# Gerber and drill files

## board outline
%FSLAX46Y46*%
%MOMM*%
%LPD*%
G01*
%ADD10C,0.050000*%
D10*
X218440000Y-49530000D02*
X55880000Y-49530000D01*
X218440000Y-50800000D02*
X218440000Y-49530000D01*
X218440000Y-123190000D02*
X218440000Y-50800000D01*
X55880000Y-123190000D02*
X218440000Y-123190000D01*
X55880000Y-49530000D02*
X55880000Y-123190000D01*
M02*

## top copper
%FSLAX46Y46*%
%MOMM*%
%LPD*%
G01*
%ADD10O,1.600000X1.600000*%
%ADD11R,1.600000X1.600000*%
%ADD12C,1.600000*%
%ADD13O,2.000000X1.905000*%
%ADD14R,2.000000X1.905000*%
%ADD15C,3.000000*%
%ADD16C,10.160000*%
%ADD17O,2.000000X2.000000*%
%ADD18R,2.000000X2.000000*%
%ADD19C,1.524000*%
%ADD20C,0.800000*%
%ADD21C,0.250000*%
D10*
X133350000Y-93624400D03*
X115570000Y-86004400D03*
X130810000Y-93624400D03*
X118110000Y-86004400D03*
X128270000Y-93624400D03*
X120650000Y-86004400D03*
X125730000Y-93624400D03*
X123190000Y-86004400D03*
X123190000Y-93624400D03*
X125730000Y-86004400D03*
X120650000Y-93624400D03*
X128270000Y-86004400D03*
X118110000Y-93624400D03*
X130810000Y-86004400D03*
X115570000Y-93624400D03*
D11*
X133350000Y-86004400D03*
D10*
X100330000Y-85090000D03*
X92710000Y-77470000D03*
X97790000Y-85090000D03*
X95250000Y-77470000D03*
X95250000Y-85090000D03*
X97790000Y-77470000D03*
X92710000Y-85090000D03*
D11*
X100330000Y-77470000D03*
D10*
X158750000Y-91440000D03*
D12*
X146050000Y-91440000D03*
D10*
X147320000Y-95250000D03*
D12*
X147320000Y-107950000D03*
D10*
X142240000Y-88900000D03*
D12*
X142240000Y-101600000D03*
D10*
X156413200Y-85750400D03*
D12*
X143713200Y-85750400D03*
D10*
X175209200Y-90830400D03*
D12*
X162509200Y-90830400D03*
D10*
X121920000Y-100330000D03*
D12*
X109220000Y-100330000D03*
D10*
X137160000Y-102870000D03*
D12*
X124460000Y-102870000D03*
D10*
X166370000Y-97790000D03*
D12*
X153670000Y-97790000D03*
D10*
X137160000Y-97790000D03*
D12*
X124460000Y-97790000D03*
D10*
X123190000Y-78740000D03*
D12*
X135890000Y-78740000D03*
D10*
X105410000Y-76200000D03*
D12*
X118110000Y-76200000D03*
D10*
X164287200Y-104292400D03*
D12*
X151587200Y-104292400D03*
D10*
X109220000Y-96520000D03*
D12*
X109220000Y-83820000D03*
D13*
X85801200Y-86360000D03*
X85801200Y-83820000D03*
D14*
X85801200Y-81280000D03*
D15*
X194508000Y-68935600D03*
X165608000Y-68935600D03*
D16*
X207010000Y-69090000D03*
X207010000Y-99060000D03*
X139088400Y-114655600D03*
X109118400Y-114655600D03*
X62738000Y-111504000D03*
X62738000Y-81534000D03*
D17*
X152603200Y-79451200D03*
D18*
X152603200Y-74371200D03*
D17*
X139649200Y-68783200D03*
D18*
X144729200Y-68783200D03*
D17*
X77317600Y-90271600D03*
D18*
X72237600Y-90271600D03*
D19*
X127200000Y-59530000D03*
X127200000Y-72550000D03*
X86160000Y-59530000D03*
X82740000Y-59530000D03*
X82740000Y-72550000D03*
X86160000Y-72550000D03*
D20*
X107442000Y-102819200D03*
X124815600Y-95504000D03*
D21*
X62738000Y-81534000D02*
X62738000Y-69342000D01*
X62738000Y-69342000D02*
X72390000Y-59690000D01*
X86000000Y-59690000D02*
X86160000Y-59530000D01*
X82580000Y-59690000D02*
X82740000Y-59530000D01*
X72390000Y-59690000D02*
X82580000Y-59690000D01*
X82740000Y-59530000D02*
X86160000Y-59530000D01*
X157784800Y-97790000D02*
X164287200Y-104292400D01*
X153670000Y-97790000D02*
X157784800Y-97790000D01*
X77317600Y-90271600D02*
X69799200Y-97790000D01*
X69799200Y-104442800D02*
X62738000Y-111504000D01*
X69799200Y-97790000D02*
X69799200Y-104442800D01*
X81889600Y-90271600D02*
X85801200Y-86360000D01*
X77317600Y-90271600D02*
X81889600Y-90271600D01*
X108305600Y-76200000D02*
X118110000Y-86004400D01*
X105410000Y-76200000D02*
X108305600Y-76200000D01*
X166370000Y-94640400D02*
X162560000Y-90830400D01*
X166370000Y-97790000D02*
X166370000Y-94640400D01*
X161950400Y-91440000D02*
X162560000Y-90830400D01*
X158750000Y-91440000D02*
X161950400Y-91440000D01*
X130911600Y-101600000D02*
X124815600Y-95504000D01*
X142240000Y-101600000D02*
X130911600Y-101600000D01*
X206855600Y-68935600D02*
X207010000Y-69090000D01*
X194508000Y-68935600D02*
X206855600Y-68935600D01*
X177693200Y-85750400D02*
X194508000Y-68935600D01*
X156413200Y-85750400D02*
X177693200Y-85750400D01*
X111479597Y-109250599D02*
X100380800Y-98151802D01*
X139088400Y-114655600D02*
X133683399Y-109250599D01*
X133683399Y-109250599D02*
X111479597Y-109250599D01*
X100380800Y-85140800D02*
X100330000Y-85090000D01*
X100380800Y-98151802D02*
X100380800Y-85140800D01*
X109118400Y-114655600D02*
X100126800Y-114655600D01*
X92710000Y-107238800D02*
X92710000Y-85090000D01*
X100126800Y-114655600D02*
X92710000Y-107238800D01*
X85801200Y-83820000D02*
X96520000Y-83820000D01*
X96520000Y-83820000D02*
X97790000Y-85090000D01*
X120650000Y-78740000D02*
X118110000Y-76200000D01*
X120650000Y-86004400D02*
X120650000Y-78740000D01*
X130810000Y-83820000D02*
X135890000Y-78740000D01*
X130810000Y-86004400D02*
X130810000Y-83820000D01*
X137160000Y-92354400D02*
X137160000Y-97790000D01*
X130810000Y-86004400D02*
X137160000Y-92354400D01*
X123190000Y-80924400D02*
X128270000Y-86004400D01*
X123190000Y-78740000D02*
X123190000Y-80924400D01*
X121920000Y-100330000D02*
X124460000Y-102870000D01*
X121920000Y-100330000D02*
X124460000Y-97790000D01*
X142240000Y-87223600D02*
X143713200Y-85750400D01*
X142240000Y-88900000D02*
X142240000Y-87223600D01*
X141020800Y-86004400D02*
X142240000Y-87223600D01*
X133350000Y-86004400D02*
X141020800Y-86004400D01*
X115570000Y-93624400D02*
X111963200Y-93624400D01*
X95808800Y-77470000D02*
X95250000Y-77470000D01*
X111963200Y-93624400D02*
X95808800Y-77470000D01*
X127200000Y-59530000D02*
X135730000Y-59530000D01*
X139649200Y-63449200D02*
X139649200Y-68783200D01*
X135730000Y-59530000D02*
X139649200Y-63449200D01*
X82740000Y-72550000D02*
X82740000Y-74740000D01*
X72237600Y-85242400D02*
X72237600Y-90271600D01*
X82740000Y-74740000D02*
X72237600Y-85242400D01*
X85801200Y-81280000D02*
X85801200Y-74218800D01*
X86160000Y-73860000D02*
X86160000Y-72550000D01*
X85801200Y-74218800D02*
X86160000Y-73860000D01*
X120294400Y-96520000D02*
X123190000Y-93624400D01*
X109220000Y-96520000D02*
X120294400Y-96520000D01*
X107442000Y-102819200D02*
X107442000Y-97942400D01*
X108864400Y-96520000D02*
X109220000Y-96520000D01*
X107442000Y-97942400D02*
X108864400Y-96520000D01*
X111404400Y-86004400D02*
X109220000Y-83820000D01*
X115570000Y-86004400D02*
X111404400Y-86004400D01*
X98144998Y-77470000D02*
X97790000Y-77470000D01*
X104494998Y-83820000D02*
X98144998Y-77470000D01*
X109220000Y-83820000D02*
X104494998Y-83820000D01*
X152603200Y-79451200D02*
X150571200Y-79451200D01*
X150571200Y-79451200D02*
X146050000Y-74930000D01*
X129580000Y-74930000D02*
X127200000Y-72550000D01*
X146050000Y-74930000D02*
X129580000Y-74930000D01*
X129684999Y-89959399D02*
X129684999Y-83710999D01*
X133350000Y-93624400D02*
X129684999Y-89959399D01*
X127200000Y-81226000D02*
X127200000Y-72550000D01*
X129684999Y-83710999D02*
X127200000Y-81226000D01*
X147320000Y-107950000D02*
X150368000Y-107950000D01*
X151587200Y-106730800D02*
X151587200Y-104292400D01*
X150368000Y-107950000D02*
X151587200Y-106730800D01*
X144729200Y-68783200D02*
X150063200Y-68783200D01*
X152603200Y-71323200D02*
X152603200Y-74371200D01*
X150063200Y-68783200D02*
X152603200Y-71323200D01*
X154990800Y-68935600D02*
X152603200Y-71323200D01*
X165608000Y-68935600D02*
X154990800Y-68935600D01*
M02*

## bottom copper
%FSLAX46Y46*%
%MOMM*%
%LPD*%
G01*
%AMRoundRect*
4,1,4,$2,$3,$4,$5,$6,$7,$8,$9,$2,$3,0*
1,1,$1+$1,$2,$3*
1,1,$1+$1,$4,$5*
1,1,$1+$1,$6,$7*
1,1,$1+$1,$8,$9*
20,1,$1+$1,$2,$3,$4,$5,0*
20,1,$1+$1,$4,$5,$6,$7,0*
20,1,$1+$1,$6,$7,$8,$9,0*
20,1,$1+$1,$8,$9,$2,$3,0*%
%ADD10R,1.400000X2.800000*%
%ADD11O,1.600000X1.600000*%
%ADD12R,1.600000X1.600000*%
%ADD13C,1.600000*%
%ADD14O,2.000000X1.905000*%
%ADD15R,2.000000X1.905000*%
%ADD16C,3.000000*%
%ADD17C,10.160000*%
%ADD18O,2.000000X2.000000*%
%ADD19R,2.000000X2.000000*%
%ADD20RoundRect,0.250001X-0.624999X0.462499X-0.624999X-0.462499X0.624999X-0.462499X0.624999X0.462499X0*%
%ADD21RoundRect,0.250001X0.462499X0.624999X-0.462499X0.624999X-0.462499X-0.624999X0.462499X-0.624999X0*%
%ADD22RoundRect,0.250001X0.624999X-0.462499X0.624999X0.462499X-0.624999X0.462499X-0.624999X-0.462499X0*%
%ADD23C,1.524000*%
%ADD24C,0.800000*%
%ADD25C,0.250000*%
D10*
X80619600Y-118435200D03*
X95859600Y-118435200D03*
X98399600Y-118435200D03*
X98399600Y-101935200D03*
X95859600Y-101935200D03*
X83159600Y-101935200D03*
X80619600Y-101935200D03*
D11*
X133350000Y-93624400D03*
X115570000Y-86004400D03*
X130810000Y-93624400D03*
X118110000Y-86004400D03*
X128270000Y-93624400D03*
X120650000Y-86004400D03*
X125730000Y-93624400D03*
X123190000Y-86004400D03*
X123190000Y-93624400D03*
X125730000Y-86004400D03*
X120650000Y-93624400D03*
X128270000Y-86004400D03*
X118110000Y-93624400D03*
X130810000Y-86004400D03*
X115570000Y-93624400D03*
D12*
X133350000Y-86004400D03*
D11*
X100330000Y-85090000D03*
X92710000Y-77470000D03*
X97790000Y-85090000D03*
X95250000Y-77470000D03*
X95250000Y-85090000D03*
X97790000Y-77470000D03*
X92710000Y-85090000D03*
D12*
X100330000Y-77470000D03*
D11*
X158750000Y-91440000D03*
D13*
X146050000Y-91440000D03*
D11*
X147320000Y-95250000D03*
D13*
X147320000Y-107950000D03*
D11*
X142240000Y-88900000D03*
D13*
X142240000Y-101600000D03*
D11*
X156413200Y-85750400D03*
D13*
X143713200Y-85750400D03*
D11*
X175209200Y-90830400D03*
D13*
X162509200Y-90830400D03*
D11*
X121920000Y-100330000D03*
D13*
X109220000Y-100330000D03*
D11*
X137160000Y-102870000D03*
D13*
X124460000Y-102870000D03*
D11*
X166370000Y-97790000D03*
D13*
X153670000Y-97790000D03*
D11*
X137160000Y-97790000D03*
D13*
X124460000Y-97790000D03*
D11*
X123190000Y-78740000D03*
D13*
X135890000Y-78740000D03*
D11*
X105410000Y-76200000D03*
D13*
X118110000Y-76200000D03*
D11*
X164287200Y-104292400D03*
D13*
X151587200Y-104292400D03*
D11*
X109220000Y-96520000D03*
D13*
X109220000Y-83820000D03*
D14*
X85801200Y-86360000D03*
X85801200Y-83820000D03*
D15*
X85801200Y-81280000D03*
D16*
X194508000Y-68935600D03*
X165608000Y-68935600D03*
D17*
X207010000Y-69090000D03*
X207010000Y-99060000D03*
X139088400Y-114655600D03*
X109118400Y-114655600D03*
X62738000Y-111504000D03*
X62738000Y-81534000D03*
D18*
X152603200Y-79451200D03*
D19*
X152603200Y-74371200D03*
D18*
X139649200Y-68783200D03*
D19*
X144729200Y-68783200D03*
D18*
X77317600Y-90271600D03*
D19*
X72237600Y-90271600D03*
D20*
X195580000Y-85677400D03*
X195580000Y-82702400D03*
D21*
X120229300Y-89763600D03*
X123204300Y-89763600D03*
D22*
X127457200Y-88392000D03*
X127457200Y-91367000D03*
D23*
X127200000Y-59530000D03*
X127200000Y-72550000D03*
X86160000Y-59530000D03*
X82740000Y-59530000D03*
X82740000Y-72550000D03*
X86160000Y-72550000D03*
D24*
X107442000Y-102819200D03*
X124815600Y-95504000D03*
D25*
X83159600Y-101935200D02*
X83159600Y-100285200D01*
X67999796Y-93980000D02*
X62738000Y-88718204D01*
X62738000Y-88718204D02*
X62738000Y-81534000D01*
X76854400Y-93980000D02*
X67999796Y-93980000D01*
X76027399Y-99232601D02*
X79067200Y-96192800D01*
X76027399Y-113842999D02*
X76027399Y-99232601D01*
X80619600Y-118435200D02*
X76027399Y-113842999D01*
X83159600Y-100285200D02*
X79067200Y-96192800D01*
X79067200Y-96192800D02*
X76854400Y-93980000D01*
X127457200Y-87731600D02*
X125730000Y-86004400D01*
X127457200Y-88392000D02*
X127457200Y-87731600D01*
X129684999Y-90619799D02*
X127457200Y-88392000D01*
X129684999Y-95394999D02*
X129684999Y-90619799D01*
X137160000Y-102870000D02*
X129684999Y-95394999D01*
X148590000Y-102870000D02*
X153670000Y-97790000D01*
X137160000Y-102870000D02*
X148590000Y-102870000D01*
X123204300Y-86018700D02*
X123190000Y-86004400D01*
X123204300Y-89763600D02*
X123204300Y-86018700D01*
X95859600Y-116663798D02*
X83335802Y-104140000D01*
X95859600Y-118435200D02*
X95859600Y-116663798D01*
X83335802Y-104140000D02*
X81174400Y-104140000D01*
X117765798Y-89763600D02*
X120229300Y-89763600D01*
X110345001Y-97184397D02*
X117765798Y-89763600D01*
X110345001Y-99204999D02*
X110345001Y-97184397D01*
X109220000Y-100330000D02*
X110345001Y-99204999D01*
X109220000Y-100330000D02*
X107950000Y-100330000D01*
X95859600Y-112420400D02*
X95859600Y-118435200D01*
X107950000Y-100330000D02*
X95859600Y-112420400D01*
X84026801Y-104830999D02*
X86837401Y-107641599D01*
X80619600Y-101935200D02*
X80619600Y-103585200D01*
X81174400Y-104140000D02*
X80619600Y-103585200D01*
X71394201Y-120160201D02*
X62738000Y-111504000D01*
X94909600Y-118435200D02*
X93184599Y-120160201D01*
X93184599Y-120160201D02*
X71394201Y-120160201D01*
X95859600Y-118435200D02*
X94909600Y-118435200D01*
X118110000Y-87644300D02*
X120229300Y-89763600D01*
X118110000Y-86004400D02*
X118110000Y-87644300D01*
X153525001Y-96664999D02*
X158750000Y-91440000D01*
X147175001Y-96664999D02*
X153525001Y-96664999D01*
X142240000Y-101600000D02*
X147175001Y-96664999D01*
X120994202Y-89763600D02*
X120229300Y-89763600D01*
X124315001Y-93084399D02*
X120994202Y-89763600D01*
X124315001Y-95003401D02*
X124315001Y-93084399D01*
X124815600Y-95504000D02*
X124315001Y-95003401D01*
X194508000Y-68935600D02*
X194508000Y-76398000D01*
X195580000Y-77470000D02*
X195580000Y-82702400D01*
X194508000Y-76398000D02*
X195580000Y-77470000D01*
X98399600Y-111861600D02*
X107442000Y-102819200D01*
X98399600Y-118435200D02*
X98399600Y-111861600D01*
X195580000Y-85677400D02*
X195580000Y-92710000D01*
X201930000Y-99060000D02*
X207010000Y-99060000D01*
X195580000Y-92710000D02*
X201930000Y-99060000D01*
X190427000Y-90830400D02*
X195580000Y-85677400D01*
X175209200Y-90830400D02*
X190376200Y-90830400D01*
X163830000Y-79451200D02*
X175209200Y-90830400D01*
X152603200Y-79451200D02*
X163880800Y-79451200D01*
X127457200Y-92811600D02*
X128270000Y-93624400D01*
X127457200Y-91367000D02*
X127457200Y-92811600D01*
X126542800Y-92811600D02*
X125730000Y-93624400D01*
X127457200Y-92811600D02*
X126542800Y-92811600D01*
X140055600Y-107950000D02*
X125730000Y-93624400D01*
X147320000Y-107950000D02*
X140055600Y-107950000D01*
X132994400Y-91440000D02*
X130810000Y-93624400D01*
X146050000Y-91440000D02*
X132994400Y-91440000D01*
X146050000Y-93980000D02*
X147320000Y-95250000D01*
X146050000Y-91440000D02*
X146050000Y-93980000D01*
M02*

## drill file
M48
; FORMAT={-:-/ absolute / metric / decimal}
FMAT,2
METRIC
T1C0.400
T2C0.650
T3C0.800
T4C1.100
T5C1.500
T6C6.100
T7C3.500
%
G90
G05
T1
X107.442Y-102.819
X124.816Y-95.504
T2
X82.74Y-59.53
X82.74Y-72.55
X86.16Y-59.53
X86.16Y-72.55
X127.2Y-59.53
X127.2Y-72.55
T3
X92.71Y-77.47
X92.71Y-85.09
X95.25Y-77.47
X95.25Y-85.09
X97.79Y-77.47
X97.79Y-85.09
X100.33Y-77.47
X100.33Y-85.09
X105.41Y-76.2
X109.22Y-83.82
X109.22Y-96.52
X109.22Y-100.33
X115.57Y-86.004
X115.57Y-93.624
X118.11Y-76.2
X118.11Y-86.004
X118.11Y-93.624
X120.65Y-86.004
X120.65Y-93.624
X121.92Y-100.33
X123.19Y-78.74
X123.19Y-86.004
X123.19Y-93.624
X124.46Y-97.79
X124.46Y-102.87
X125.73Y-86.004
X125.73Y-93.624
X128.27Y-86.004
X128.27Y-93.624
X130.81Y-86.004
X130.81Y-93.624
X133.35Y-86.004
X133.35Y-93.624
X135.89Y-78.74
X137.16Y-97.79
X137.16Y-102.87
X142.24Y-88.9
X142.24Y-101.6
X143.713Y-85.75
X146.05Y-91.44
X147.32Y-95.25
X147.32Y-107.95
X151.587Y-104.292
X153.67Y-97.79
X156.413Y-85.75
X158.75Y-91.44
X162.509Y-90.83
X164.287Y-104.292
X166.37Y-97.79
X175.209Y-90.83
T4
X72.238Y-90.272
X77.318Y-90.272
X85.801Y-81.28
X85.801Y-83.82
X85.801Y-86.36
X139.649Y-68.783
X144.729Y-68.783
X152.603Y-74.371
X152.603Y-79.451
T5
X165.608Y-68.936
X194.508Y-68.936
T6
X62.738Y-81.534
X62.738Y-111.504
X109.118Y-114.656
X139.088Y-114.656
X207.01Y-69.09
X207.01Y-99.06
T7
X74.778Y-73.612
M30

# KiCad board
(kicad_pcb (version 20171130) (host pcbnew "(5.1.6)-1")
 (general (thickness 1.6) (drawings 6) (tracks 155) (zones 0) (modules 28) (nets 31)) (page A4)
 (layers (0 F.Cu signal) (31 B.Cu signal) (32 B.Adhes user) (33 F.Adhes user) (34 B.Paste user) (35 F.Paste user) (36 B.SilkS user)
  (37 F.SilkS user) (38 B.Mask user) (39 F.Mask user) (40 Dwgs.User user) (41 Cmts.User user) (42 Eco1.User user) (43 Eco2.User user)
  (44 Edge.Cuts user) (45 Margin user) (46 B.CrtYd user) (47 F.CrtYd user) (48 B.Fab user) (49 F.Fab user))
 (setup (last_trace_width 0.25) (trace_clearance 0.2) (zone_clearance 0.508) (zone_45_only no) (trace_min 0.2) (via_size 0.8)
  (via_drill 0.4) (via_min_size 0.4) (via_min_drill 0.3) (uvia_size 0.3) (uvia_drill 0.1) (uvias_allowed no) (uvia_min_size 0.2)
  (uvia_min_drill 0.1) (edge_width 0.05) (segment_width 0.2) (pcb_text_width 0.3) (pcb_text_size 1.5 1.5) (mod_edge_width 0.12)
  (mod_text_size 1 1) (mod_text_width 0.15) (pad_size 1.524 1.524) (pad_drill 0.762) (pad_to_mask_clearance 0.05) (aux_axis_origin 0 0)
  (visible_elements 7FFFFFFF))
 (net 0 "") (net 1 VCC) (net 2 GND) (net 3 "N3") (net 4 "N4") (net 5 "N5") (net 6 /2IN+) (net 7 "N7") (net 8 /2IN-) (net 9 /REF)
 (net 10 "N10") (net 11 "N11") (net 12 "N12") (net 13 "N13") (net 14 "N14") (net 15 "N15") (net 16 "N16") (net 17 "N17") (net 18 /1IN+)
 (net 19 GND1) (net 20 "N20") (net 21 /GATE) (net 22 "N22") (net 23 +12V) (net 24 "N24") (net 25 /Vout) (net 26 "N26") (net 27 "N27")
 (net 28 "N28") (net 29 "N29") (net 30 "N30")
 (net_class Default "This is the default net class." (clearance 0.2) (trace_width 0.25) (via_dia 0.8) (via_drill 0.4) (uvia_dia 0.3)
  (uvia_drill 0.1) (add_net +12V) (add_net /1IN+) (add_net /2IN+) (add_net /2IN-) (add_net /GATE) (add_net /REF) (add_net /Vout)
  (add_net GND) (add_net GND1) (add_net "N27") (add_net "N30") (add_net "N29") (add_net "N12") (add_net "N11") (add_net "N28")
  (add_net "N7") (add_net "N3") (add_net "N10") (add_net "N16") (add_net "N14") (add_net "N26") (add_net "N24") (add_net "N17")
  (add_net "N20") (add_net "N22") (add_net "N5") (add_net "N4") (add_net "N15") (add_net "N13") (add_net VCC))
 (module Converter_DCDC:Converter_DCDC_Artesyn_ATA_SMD (layer B.Cu) (at 89.5096 110.1852 270)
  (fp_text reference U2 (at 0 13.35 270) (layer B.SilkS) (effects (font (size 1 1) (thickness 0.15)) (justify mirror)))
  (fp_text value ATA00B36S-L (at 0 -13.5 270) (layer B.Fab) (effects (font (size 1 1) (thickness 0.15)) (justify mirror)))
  (pad 16 smd rect (at 8.25 8.89 270) (size 2.8 1.4) (layers B.Cu B.Paste B.Mask) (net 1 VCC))
  (pad 10 smd rect (at 8.25 -6.35 270) (size 2.8 1.4) (layers B.Cu B.Paste B.Mask) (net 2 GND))
  (pad 9 smd rect (at 8.25 -8.89 270) (size 2.8 1.4) (layers B.Cu B.Paste B.Mask) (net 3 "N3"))
  (pad 8 smd rect (at -8.25 -8.89 270) (size 2.8 1.4) (layers B.Cu B.Paste B.Mask) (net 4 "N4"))
  (pad 7 smd rect (at -8.25 -6.35 270) (size 2.8 1.4) (layers B.Cu B.Paste B.Mask) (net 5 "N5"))
  (pad 2 smd rect (at -8.25 6.35 270) (size 2.8 1.4) (layers B.Cu B.Paste B.Mask) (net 1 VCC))
  (pad 1 smd rect (at -8.25 8.89 270) (size 2.8 1.4) (layers B.Cu B.Paste B.Mask) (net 2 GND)))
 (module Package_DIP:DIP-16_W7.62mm (layer F.Cu) (at 133.35 86.0044 270)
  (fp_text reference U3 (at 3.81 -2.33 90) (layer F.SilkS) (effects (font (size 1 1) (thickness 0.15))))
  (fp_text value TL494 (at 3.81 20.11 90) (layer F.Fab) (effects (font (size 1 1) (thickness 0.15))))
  (pad 16 thru_hole oval (at 7.62 0 270) (size 1.6 1.6) (drill 0.8) (layers *.Cu *.Mask) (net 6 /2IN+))
  (pad 8 thru_hole oval (at 0 17.78 270) (size 1.6 1.6) (drill 0.8) (layers *.Cu *.Mask) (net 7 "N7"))
  (pad 15 thru_hole oval (at 7.62 2.54 270) (size 1.6 1.6) (drill 0.8) (layers *.Cu *.Mask) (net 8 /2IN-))
  (pad 7 thru_hole oval (at 0 15.24 270) (size 1.6 1.6) (drill 0.8) (layers *.Cu *.Mask) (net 2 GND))
  (pad 14 thru_hole oval (at 7.62 5.08 270) (size 1.6 1.6) (drill 0.8) (layers *.Cu *.Mask) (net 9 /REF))
  (pad 6 thru_hole oval (at 0 12.7 270) (size 1.6 1.6) (drill 0.8) (layers *.Cu *.Mask) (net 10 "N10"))
  (pad 13 thru_hole oval (at 7.62 7.62 270) (size 1.6 1.6) (drill 0.8) (layers *.Cu *.Mask) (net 9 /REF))
  (pad 5 thru_hole oval (at 0 10.16 270) (size 1.6 1.6) (drill 0.8) (layers *.Cu *.Mask) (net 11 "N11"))
  (pad 12 thru_hole oval (at 7.62 10.16 270) (size 1.6 1.6) (drill 0.8) (layers *.Cu *.Mask) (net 3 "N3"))
  (pad 4 thru_hole oval (at 0 7.62 270) (size 1.6 1.6) (drill 0.8) (layers *.Cu *.Mask) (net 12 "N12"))
  (pad 11 thru_hole oval (at 7.62 12.7 270) (size 1.6 1.6) (drill 0.8) (layers *.Cu *.Mask) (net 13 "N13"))
  (pad 3 thru_hole oval (at 0 5.08 270) (size 1.6 1.6) (drill 0.8) (layers *.Cu *.Mask) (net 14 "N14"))
  (pad 10 thru_hole oval (at 7.62 15.24 270) (size 1.6 1.6) (drill 0.8) (layers *.Cu *.Mask) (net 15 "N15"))
  (pad 2 thru_hole oval (at 0 2.54 270) (size 1.6 1.6) (drill 0.8) (layers *.Cu *.Mask) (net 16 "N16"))
  (pad 9 thru_hole oval (at 7.62 17.78 270) (size 1.6 1.6) (drill 0.8) (layers *.Cu *.Mask) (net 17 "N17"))
  (pad 1 thru_hole rect (at 0 0 270) (size 1.6 1.6) (drill 0.8) (layers *.Cu *.Mask) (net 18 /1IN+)))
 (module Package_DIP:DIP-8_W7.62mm (layer F.Cu) (at 100.33 77.47 270)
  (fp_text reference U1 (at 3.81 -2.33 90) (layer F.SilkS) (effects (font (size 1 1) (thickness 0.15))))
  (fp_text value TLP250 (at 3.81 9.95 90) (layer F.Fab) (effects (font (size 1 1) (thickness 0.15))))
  (pad 8 thru_hole oval (at 7.62 0 270) (size 1.6 1.6) (drill 0.8) (layers *.Cu *.Mask) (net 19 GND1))
  (pad 4 thru_hole oval (at 0 7.62 270) (size 1.6 1.6) (drill 0.8) (layers *.Cu *.Mask) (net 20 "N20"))
  (pad 7 thru_hole oval (at 7.62 2.54 270) (size 1.6 1.6) (drill 0.8) (layers *.Cu *.Mask) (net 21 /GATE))
  (pad 3 thru_hole oval (at 0 5.08 270) (size 1.6 1.6) (drill 0.8) (layers *.Cu *.Mask) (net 17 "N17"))
  (pad 6 thru_hole oval (at 7.62 5.08 270) (size 1.6 1.6) (drill 0.8) (layers *.Cu *.Mask) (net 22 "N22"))
  (pad 2 thru_hole oval (at 0 2.54 270) (size 1.6 1.6) (drill 0.8) (layers *.Cu *.Mask) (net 7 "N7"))
  (pad 5 thru_hole oval (at 7.62 7.62 270) (size 1.6 1.6) (drill 0.8) (layers *.Cu *.Mask) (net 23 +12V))
  (pad 1 thru_hole rect (at 0 0 270) (size 1.6 1.6) (drill 0.8) (layers *.Cu *.Mask) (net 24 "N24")))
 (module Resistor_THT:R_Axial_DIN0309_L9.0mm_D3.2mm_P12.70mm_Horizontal (layer F.Cu) (at 146.05 91.44)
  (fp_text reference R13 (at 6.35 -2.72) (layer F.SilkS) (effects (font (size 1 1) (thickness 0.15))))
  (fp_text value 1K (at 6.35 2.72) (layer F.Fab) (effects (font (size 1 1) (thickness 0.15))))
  (pad 2 thru_hole oval (at 12.7 0) (size 1.6 1.6) (drill 0.8) (layers *.Cu *.Mask) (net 2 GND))
  (pad 1 thru_hole circle (at 0 0) (size 1.6 1.6) (drill 0.8) (layers *.Cu *.Mask) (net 8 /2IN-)))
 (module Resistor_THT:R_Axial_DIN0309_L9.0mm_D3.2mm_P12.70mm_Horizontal (layer F.Cu) (at 147.32 107.95 90)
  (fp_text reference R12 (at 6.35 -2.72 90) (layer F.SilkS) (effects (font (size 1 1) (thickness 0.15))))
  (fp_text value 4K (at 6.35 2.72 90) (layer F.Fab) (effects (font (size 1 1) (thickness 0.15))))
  (pad 2 thru_hole oval (at 12.7 0 90) (size 1.6 1.6) (drill 0.8) (layers *.Cu *.Mask) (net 8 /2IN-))
  (pad 1 thru_hole circle (at 0 0 90) (size 1.6 1.6) (drill 0.8) (layers *.Cu *.Mask) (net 9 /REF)))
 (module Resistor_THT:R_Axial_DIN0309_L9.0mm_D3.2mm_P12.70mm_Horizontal (layer F.Cu) (at 142.24 101.6 90)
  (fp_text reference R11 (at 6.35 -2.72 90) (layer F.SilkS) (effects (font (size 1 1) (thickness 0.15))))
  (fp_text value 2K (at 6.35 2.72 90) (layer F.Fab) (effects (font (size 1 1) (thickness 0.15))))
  (pad 2 thru_hole oval (at 12.7 0 90) (size 1.6 1.6) (drill 0.8) (layers *.Cu *.Mask) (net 18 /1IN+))
  (pad 1 thru_hole circle (at 0 0 90) (size 1.6 1.6) (drill 0.8) (layers *.Cu *.Mask) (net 2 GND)))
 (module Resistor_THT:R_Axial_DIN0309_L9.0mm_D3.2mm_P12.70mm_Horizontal (layer F.Cu) (at 143.7132 85.7504)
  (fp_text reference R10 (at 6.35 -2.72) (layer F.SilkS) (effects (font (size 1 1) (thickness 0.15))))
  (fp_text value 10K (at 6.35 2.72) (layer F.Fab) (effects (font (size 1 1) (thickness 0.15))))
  (pad 2 thru_hole oval (at 12.7 0) (size 1.6 1.6) (drill 0.8) (layers *.Cu *.Mask) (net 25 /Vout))
  (pad 1 thru_hole circle (at 0 0) (size 1.6 1.6) (drill 0.8) (layers *.Cu *.Mask) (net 18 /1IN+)))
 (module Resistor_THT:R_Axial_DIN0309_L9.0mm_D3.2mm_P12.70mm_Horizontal (layer F.Cu) (at 162.5092 90.8304)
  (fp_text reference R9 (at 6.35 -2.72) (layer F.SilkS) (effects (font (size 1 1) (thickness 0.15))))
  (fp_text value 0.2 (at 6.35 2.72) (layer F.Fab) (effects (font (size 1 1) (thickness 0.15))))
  (pad 2 thru_hole oval (at 12.7 0) (size 1.6 1.6) (drill 0.8) (layers *.Cu *.Mask) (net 6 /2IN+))
  (pad 1 thru_hole circle (at 0 0) (size 1.6 1.6) (drill 0.8) (layers *.Cu *.Mask) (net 2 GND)))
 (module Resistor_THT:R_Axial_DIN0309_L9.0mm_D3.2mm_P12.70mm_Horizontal (layer F.Cu) (at 109.22 100.33)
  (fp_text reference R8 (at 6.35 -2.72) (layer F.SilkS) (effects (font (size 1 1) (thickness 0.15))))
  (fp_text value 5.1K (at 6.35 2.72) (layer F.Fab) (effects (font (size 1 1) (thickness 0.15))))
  (pad 2 thru_hole oval (at 12.7 0) (size 1.6 1.6) (drill 0.8) (layers *.Cu *.Mask) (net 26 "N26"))
  (pad 1 thru_hole circle (at 0 0) (size 1.6 1.6) (drill 0.8) (layers *.Cu *.Mask) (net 2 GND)))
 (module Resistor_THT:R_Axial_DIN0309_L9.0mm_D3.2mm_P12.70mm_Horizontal (layer F.Cu) (at 124.46 102.87)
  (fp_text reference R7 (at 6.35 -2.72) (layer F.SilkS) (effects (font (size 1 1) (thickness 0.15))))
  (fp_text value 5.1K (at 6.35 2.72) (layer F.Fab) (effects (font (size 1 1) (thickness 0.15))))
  (pad 2 thru_hole oval (at 12.7 0) (size 1.6 1.6) (drill 0.8) (layers *.Cu *.Mask) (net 12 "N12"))
  (pad 1 thru_hole circle (at 0 0) (size 1.6 1.6) (drill 0.8) (layers *.Cu *.Mask) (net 26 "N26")))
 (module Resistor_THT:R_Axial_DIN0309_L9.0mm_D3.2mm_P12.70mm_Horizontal (layer F.Cu) (at 153.67 97.79)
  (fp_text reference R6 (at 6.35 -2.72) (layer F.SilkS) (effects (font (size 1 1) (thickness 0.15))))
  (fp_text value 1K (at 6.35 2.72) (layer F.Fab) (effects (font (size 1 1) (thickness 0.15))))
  (pad 2 thru_hole oval (at 12.7 0) (size 1.6 1.6) (drill 0.8) (layers *.Cu *.Mask) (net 2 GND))
  (pad 1 thru_hole circle (at 0 0) (size 1.6 1.6) (drill 0.8) (layers *.Cu *.Mask) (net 12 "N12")))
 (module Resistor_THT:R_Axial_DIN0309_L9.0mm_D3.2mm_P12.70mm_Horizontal (layer F.Cu) (at 124.46 97.79)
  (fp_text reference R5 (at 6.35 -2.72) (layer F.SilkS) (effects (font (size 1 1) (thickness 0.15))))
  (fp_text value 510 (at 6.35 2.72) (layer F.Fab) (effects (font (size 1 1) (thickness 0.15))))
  (pad 2 thru_hole oval (at 12.7 0) (size 1.6 1.6) (drill 0.8) (layers *.Cu *.Mask) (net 16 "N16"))
  (pad 1 thru_hole circle (at 0 0) (size 1.6 1.6) (drill 0.8) (layers *.Cu *.Mask) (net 26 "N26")))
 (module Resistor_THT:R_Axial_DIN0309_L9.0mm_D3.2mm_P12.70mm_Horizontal (layer F.Cu) (at 135.89 78.74 180)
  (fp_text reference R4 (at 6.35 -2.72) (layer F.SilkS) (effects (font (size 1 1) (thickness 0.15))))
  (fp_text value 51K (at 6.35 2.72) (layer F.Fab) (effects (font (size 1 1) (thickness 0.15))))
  (pad 2 thru_hole oval (at 12.7 0 180) (size 1.6 1.6) (drill 0.8) (layers *.Cu *.Mask) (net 14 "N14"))
  (pad 1 thru_hole circle (at 0 0 180) (size 1.6 1.6) (drill 0.8) (layers *.Cu *.Mask) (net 16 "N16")))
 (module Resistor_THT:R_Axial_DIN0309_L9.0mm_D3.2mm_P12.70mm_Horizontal (layer F.Cu) (at 118.11 76.2 180)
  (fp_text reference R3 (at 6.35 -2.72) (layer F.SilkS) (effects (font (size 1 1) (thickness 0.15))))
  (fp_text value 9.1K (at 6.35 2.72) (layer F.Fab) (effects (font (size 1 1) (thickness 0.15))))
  (pad 2 thru_hole oval (at 12.7 0 180) (size 1.6 1.6) (drill 0.8) (layers *.Cu *.Mask) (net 2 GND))
  (pad 1 thru_hole circle (at 0 0 180) (size 1.6 1.6) (drill 0.8) (layers *.Cu *.Mask) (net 10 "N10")))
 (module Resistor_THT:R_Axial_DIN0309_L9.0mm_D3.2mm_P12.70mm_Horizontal (layer F.Cu) (at 151.5872 104.2924)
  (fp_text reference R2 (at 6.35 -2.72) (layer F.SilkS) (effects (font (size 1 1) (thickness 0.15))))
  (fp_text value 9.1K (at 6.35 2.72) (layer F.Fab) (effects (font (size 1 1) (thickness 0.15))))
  (pad 2 thru_hole oval (at 12.7 0) (size 1.6 1.6) (drill 0.8) (layers *.Cu *.Mask) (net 12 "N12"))
  (pad 1 thru_hole circle (at 0 0) (size 1.6 1.6) (drill 0.8) (layers *.Cu *.Mask) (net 9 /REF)))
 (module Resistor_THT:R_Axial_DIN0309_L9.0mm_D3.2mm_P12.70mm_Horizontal (layer B.Cu) (at 109.22 83.82 270)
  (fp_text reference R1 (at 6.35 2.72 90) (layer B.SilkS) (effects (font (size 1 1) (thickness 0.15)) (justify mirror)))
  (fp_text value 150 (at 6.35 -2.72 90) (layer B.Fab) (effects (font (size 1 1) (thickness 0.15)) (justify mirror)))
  (pad 2 thru_hole oval (at 12.7 0 270) (size 1.6 1.6) (drill 0.8) (layers *.Cu *.Mask) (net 3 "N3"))
  (pad 1 thru_hole circle (at 0 0 270) (size 1.6 1.6) (drill 0.8) (layers *.Cu *.Mask) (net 7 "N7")))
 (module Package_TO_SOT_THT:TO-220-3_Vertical (layer F.Cu) (at 85.8012 81.28 270)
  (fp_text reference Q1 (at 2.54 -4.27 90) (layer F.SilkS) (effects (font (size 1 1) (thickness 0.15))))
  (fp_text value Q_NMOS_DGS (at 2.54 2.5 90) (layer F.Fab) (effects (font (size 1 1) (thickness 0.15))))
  (pad 3 thru_hole oval (at 5.08 0 270) (size 1.905 2) (drill 1.1) (layers *.Cu *.Mask) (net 2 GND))
  (pad 2 thru_hole oval (at 2.54 0 270) (size 1.905 2) (drill 1.1) (layers *.Cu *.Mask) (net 21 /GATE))
  (pad 1 thru_hole rect (at 0 0 270) (size 1.905 2) (drill 1.1) (layers *.Cu *.Mask) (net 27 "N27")))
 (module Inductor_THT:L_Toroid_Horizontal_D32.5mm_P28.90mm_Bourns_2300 (layer F.Cu) (at 165.608 68.9356)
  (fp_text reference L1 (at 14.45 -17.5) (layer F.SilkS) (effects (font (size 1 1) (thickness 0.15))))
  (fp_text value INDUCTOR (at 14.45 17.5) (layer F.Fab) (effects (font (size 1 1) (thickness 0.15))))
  (pad 2 thru_hole circle (at 28.9 0) (size 3 3) (drill 1.5) (layers *.Cu *.Mask) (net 25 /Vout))
  (pad 1 thru_hole circle (at 0 0) (size 3 3) (drill 1.5) (layers *.Cu *.Mask) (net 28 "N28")))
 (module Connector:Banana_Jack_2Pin (layer F.Cu) (at 207.01 99.06 90)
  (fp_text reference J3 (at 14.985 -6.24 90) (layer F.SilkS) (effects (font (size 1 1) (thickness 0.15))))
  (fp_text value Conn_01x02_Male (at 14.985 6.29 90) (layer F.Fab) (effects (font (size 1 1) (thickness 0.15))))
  (pad 2 thru_hole circle (at 29.97 0 90) (size 10.16 10.16) (drill 6.1) (layers *.Cu *.Mask) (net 25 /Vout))
  (pad 1 thru_hole circle (at 0 0 90) (size 10.16 10.16) (drill 6.1) (layers *.Cu *.Mask) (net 6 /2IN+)))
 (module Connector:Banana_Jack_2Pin (layer F.Cu) (at 109.1184 114.6556)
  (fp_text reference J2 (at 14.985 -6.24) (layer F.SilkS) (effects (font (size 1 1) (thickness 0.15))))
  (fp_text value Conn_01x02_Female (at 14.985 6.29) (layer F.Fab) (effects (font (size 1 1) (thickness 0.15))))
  (pad 2 thru_hole circle (at 29.97 0) (size 10.16 10.16) (drill 6.1) (layers *.Cu *.Mask) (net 19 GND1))
  (pad 1 thru_hole circle (at 0 0) (size 10.16 10.16) (drill 6.1) (layers *.Cu *.Mask) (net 23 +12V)))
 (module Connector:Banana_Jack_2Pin (layer F.Cu) (at 62.738 81.534 270)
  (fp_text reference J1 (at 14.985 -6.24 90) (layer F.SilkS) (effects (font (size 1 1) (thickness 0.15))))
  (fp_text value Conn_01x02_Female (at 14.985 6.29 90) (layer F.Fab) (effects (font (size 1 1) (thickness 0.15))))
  (pad 2 thru_hole circle (at 29.97 0 270) (size 10.16 10.16) (drill 6.1) (layers *.Cu *.Mask) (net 2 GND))
  (pad 1 thru_hole circle (at 0 0 270) (size 10.16 10.16) (drill 6.1) (layers *.Cu *.Mask) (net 1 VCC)))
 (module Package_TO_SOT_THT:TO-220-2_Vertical (layer F.Cu) (at 152.6032 74.3712 270)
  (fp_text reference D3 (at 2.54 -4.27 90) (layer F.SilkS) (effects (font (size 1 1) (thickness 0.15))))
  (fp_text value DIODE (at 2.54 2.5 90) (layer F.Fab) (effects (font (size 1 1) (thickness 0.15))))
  (pad 2 thru_hole oval (at 5.08 0 270) (size 2 2) (drill 1.1) (layers *.Cu *.Mask) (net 6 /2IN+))
  (pad 1 thru_hole rect (at 0 0 270) (size 2 2) (drill 1.1) (layers *.Cu *.Mask) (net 28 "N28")))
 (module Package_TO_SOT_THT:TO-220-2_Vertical (layer F.Cu) (at 144.7292 68.7832 180)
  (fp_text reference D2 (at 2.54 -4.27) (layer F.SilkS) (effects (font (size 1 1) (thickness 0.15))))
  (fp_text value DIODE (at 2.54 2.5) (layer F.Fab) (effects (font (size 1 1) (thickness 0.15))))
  (pad 2 thru_hole oval (at 5.08 0 180) (size 2 2) (drill 1.1) (layers *.Cu *.Mask) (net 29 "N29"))
  (pad 1 thru_hole rect (at 0 0 180) (size 2 2) (drill 1.1) (layers *.Cu *.Mask) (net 28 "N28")))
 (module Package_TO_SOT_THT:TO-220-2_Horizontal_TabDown (layer F.Cu) (at 72.2376 90.2716)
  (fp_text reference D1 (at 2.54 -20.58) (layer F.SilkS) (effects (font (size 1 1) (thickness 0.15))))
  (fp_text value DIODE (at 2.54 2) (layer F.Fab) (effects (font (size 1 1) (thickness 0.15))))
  (pad 2 thru_hole oval (at 5.08 0) (size 2 2) (drill 1.1) (layers *.Cu *.Mask) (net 2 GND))
  (pad 1 thru_hole rect (at 0 0) (size 2 2) (drill 1.1) (layers *.Cu *.Mask) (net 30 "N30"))
  (pad "" np_thru_hole oval (at 2.54 -16.66) (size 3.5 3.5) (drill 3.5) (layers *.Cu *.Mask)))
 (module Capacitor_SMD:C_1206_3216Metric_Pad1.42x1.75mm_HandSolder (layer B.Cu) (at 195.58 84.1899 270)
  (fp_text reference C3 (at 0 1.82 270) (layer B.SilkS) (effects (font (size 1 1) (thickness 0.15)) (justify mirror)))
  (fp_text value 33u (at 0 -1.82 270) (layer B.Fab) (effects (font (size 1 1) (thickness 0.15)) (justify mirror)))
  (pad 2 smd roundrect (at 1.4875 0 270) (size 1.425 1.75) (layers B.Cu B.Paste B.Mask) (roundrect_rratio 0.175439) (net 6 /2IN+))
  (pad 1 smd roundrect (at -1.4875 0 270) (size 1.425 1.75) (layers B.Cu B.Paste B.Mask) (roundrect_rratio 0.175439) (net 25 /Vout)))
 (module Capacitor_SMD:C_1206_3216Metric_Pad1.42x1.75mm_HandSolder (layer B.Cu) (at 121.7168 89.7636 180)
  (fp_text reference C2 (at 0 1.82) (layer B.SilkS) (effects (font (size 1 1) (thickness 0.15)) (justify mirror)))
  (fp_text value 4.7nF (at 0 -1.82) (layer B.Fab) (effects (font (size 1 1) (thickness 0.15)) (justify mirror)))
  (pad 2 smd roundrect (at 1.4875 0 180) (size 1.425 1.75) (layers B.Cu B.Paste B.Mask) (roundrect_rratio 0.175439) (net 2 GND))
  (pad 1 smd roundrect (at -1.4875 0 180) (size 1.425 1.75) (layers B.Cu B.Paste B.Mask) (roundrect_rratio 0.175439) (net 11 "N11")))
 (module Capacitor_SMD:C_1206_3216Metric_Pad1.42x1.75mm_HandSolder (layer B.Cu) (at 127.4572 89.8795 90)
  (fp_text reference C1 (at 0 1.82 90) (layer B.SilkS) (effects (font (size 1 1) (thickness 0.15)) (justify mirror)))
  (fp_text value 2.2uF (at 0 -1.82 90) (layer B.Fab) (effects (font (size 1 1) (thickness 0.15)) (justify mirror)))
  (pad 2 smd roundrect (at 1.4875 0 90) (size 1.425 1.75) (layers B.Cu B.Paste B.Mask) (roundrect_rratio 0.175439) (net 12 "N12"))
  (pad 1 smd roundrect (at -1.4875 0 90) (size 1.425 1.75) (layers B.Cu B.Paste B.Mask) (roundrect_rratio 0.175439) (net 9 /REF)))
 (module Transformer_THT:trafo (layer F.Cu) (at 106.68 66.04 90)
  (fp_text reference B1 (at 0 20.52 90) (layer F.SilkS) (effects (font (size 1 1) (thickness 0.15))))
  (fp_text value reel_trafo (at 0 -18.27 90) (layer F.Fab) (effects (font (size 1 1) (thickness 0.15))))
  (pad 6 thru_hole circle (at 6.51 20.52 90) (size 1.524 1.524) (drill 0.65) (layers *.Cu *.Mask) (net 29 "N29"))
  (pad 5 thru_hole circle (at -6.51 20.52 90) (size 1.524 1.524) (drill 0.65) (layers *.Cu *.Mask) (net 6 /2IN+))
  (pad 4 thru_hole circle (at 6.51 -20.52 90) (size 1.524 1.524) (drill 0.65) (layers *.Cu *.Mask) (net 1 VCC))
  (pad 3 thru_hole circle (at 6.51 -23.94 90) (size 1.524 1.524) (drill 0.65) (layers *.Cu *.Mask) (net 1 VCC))
  (pad 2 thru_hole circle (at -6.51 -23.94 90) (size 1.524 1.524) (drill 0.65) (layers *.Cu *.Mask) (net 30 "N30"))
  (pad 1 thru_hole circle (at -6.51 -20.52 90) (size 1.524 1.524) (drill 0.65) (layers *.Cu *.Mask) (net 27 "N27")))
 (gr_line (start 218.44 49.53) (end 55.88 49.53) (layer Edge.Cuts) (width 0.05))
 (gr_line (start 218.44 50.8) (end 218.44 49.53) (layer Edge.Cuts) (width 0.05))
 (gr_line (start 218.44 123.19) (end 218.44 50.8) (layer Edge.Cuts) (width 0.05))
 (gr_line (start 55.88 123.19) (end 218.44 123.19) (layer Edge.Cuts) (width 0.05))
 (gr_line (start 55.88 49.53) (end 55.88 123.19) (layer Edge.Cuts) (width 0.05))
 (via (at 107.442 102.8192) (size 0.8) (drill 0.4) (layers F.Cu B.Cu) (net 3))
 (via (at 124.8156 95.504) (size 0.8) (drill 0.4) (layers F.Cu B.Cu) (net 2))
 (segment (start 62.738 81.534) (end 62.738 69.342) (width 0.25) (layer F.Cu) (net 1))
 (segment (start 62.738 69.342) (end 72.39 59.69) (width 0.25) (layer F.Cu) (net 1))
 (segment (start 86 59.69) (end 86.16 59.53) (width 0.25) (layer F.Cu) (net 1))
 (segment (start 82.58 59.69) (end 82.74 59.53) (width 0.25) (layer F.Cu) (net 1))
 (segment (start 72.39 59.69) (end 82.58 59.69) (width 0.25) (layer F.Cu) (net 1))
 (segment (start 82.74 59.53) (end 86.16 59.53) (width 0.25) (layer F.Cu) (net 1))
 (segment (start 83.1596 101.9352) (end 83.1596 100.2852) (width 0.25) (layer B.Cu) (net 1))
 (segment (start 67.999796 93.98) (end 62.738 88.718204) (width 0.25) (layer B.Cu) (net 1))
 (segment (start 62.738 88.718204) (end 62.738 81.534) (width 0.25) (layer B.Cu) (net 1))
 (segment (start 76.8544 93.98) (end 67.999796 93.98) (width 0.25) (layer B.Cu) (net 1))
 (segment (start 76.027399 99.232601) (end 79.0672 96.1928) (width 0.25) (layer B.Cu) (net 1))
 (segment (start 76.027399 113.842999) (end 76.027399 99.232601) (width 0.25) (layer B.Cu) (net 1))
 (segment (start 80.6196 118.4352) (end 76.027399 113.842999) (width 0.25) (layer B.Cu) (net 1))
 (segment (start 83.1596 100.2852) (end 79.0672 96.1928) (width 0.25) (layer B.Cu) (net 1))
 (segment (start 79.0672 96.1928) (end 76.8544 93.98) (width 0.25) (layer B.Cu) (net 1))
 (segment (start 127.4572 87.7316) (end 125.73 86.0044) (width 0.25) (layer B.Cu) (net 12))
 (segment (start 127.4572 88.392) (end 127.4572 87.7316) (width 0.25) (layer B.Cu) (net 12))
 (segment (start 157.7848 97.79) (end 164.2872 104.2924) (width 0.25) (layer F.Cu) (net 12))
 (segment (start 153.67 97.79) (end 157.7848 97.79) (width 0.25) (layer F.Cu) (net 12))
 (segment (start 129.684999 90.619799) (end 127.4572 88.392) (width 0.25) (layer B.Cu) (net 12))
 (segment (start 129.684999 95.394999) (end 129.684999 90.619799) (width 0.25) (layer B.Cu) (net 12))
 (segment (start 137.16 102.87) (end 129.684999 95.394999) (width 0.25) (layer B.Cu) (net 12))
 (segment (start 148.59 102.87) (end 153.67 97.79) (width 0.25) (layer B.Cu) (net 12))
 (segment (start 137.16 102.87) (end 148.59 102.87) (width 0.25) (layer B.Cu) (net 12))
 (segment (start 123.2043 86.0187) (end 123.19 86.0044) (width 0.25) (layer B.Cu) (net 11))
 (segment (start 123.2043 89.7636) (end 123.2043 86.0187) (width 0.25) (layer B.Cu) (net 11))
 (segment (start 77.3176 90.2716) (end 69.7992 97.79) (width 0.25) (layer F.Cu) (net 2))
 (segment (start 69.7992 104.4428) (end 62.738 111.504) (width 0.25) (layer F.Cu) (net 2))
 (segment (start 69.7992 97.79) (end 69.7992 104.4428) (width 0.25) (layer F.Cu) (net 2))
 (segment (start 81.8896 90.2716) (end 85.8012 86.36) (width 0.25) (layer F.Cu) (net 2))
 (segment (start 77.3176 90.2716) (end 81.8896 90.2716) (width 0.25) (layer F.Cu) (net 2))
 (segment (start 95.8596 116.663798) (end 83.335802 104.14) (width 0.25) (layer B.Cu) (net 2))
 (segment (start 95.8596 118.4352) (end 95.8596 116.663798) (width 0.25) (layer B.Cu) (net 2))
 (segment (start 83.335802 104.14) (end 81.1744 104.14) (width 0.25) (layer B.Cu) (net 2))
 (segment (start 117.765798 89.7636) (end 120.2293 89.7636) (width 0.25) (layer B.Cu) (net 2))
 (segment (start 110.345001 97.184397) (end 117.765798 89.7636) (width 0.25) (layer B.Cu) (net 2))
 (segment (start 110.345001 99.204999) (end 110.345001 97.184397) (width 0.25) (layer B.Cu) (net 2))
 (segment (start 109.22 100.33) (end 110.345001 99.204999) (width 0.25) (layer B.Cu) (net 2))
 (segment (start 109.22 100.33) (end 107.95 100.33) (width 0.25) (layer B.Cu) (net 2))
 (segment (start 95.8596 112.4204) (end 95.8596 118.4352) (width 0.25) (layer B.Cu) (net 2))
 (segment (start 107.95 100.33) (end 95.8596 112.4204) (width 0.25) (layer B.Cu) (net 2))
 (segment (start 84.026801 104.830999) (end 86.837401 107.641599) (width 0.25) (layer B.Cu) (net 2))
 (segment (start 80.6196 101.9352) (end 80.6196 103.5852) (width 0.25) (layer B.Cu) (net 2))
 (segment (start 81.1744 104.14) (end 80.6196 103.5852) (width 0.25) (layer B.Cu) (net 2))
 (segment (start 71.394201 120.160201) (end 62.738 111.504) (width 0.25) (layer B.Cu) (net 2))
 (segment (start 94.9096 118.4352) (end 93.184599 120.160201) (width 0.25) (layer B.Cu) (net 2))
 (segment (start 93.184599 120.160201) (end 71.394201 120.160201) (width 0.25) (layer B.Cu) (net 2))
 (segment (start 95.8596 118.4352) (end 94.9096 118.4352) (width 0.25) (layer B.Cu) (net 2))
 (segment (start 118.11 87.6443) (end 120.2293 89.7636) (width 0.25) (layer B.Cu) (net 2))
 (segment (start 118.11 86.0044) (end 118.11 87.6443) (width 0.25) (layer B.Cu) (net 2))
 (segment (start 108.3056 76.2) (end 118.11 86.0044) (width 0.25) (layer F.Cu) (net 2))
 (segment (start 105.41 76.2) (end 108.3056 76.2) (width 0.25) (layer F.Cu) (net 2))
 (segment (start 166.37 94.6404) (end 162.56 90.8304) (width 0.25) (layer F.Cu) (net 2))
 (segment (start 166.37 97.79) (end 166.37 94.6404) (width 0.25) (layer F.Cu) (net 2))
 (segment (start 161.9504 91.44) (end 162.56 90.8304) (width 0.25) (layer F.Cu) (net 2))
 (segment (start 158.75 91.44) (end 161.9504 91.44) (width 0.25) (layer F.Cu) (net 2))
 (segment (start 153.525001 96.664999) (end 158.75 91.44) (width 0.25) (layer B.Cu) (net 2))
 (segment (start 147.175001 96.664999) (end 153.525001 96.664999) (width 0.25) (layer B.Cu) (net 2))
 (segment (start 142.24 101.6) (end 147.175001 96.664999) (width 0.25) (layer B.Cu) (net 2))
 (segment (start 130.9116 101.6) (end 124.8156 95.504) (width 0.25) (layer F.Cu) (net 2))
 (segment (start 142.24 101.6) (end 130.9116 101.6) (width 0.25) (layer F.Cu) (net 2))
 (segment (start 120.994202 89.7636) (end 120.2293 89.7636) (width 0.25) (layer B.Cu) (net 2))
 (segment (start 124.315001 93.084399) (end 120.994202 89.7636) (width 0.25) (layer B.Cu) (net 2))
 (segment (start 124.315001 95.003401) (end 124.315001 93.084399) (width 0.25) (layer B.Cu) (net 2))
 (segment (start 124.8156 95.504) (end 124.315001 95.003401) (width 0.25) (layer B.Cu) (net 2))
 (segment (start 206.8556 68.9356) (end 207.01 69.09) (width 0.25) (layer F.Cu) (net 25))
 (segment (start 194.508 68.9356) (end 206.8556 68.9356) (width 0.25) (layer F.Cu) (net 25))
 (segment (start 194.508 68.9356) (end 194.508 76.398) (width 0.25) (layer B.Cu) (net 25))
 (segment (start 195.58 77.47) (end 195.58 82.7024) (width 0.25) (layer B.Cu) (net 25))
 (segment (start 194.508 76.398) (end 195.58 77.47) (width 0.25) (layer B.Cu) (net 25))
 (segment (start 177.6932 85.7504) (end 194.508 68.9356) (width 0.25) (layer F.Cu) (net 25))
 (segment (start 156.4132 85.7504) (end 177.6932 85.7504) (width 0.25) (layer F.Cu) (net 25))
 (segment (start 111.479597 109.250599) (end 100.3808 98.151802) (width 0.25) (layer F.Cu) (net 19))
 (segment (start 139.0884 114.6556) (end 133.683399 109.250599) (width 0.25) (layer F.Cu) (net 19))
 (segment (start 133.683399 109.250599) (end 111.479597 109.250599) (width 0.25) (layer F.Cu) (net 19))
 (segment (start 100.3808 85.1408) (end 100.33 85.09) (width 0.25) (layer F.Cu) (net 19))
 (segment (start 100.3808 98.151802) (end 100.3808 85.1408) (width 0.25) (layer F.Cu) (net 19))
 (segment (start 109.1184 114.6556) (end 100.1268 114.6556) (width 0.25) (layer F.Cu) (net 23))
 (segment (start 92.71 107.2388) (end 92.71 85.09) (width 0.25) (layer F.Cu) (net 23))
 (segment (start 100.1268 114.6556) (end 92.71 107.2388) (width 0.25) (layer F.Cu) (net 23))
 (segment (start 85.8012 83.82) (end 96.52 83.82) (width 0.25) (layer F.Cu) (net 21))
 (segment (start 96.52 83.82) (end 97.79 85.09) (width 0.25) (layer F.Cu) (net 21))
 (segment (start 120.65 78.74) (end 118.11 76.2) (width 0.25) (layer F.Cu) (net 10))
 (segment (start 120.65 86.0044) (end 120.65 78.74) (width 0.25) (layer F.Cu) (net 10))
 (segment (start 130.81 83.82) (end 135.89 78.74) (width 0.25) (layer F.Cu) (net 16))
 (segment (start 130.81 86.0044) (end 130.81 83.82) (width 0.25) (layer F.Cu) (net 16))
 (segment (start 137.16 92.3544) (end 137.16 97.79) (width 0.25) (layer F.Cu) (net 16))
 (segment (start 130.81 86.0044) (end 137.16 92.3544) (width 0.25) (layer F.Cu) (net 16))
 (segment (start 123.19 80.9244) (end 128.27 86.0044) (width 0.25) (layer F.Cu) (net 14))
 (segment (start 123.19 78.74) (end 123.19 80.9244) (width 0.25) (layer F.Cu) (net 14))
 (segment (start 121.92 100.33) (end 124.46 102.87) (width 0.25) (layer F.Cu) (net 26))
 (segment (start 121.92 100.33) (end 124.46 97.79) (width 0.25) (layer F.Cu) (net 26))
 (segment (start 142.24 87.2236) (end 143.7132 85.7504) (width 0.25) (layer F.Cu) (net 18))
 (segment (start 142.24 88.9) (end 142.24 87.2236) (width 0.25) (layer F.Cu) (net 18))
 (segment (start 141.0208 86.0044) (end 142.24 87.2236) (width 0.25) (layer F.Cu) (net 18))
 (segment (start 133.35 86.0044) (end 141.0208 86.0044) (width 0.25) (layer F.Cu) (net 18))
 (segment (start 115.57 93.6244) (end 111.9632 93.6244) (width 0.25) (layer F.Cu) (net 17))
 (segment (start 95.8088 77.47) (end 95.25 77.47) (width 0.25) (layer F.Cu) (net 17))
 (segment (start 111.9632 93.6244) (end 95.8088 77.47) (width 0.25) (layer F.Cu) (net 17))
 (segment (start 127.2 59.53) (end 135.73 59.53) (width 0.25) (layer F.Cu) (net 29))
 (segment (start 139.6492 63.4492) (end 139.6492 68.7832) (width 0.25) (layer F.Cu) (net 29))
 (segment (start 135.73 59.53) (end 139.6492 63.4492) (width 0.25) (layer F.Cu) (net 29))
 (segment (start 82.74 72.55) (end 82.74 74.74) (width 0.25) (layer F.Cu) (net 30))
 (segment (start 72.2376 85.2424) (end 72.2376 90.2716) (width 0.25) (layer F.Cu) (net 30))
 (segment (start 82.74 74.74) (end 72.2376 85.2424) (width 0.25) (layer F.Cu) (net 30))
 (segment (start 85.8012 81.28) (end 85.8012 74.2188) (width 0.25) (layer F.Cu) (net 27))
 (segment (start 86.16 73.86) (end 86.16 72.55) (width 0.25) (layer F.Cu) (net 27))
 (segment (start 85.8012 74.2188) (end 86.16 73.86) (width 0.25) (layer F.Cu) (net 27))
 (segment (start 120.2944 96.52) (end 123.19 93.6244) (width 0.25) (layer F.Cu) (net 3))
 (segment (start 109.22 96.52) (end 120.2944 96.52) (width 0.25) (layer F.Cu) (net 3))
 (segment (start 98.3996 111.8616) (end 107.442 102.8192) (width 0.25) (layer B.Cu) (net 3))
 (segment (start 98.3996 118.4352) (end 98.3996 111.8616) (width 0.25) (layer B.Cu) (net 3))
 (segment (start 107.442 102.8192) (end 107.442 97.9424) (width 0.25) (layer F.Cu) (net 3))
 (segment (start 108.8644 96.52) (end 109.22 96.52) (width 0.25) (layer F.Cu) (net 3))
 (segment (start 107.442 97.9424) (end 108.8644 96.52) (width 0.25) (layer F.Cu) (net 3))
 (segment (start 111.4044 86.0044) (end 109.22 83.82) (width 0.25) (layer F.Cu) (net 7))
 (segment (start 115.57 86.0044) (end 111.4044 86.0044) (width 0.25) (layer F.Cu) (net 7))
 (segment (start 98.144998 77.47) (end 97.79 77.47) (width 0.25) (layer F.Cu) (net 7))
 (segment (start 104.494998 83.82) (end 98.144998 77.47) (width 0.25) (layer F.Cu) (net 7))
 (segment (start 109.22 83.82) (end 104.494998 83.82) (width 0.25) (layer F.Cu) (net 7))
 (segment (start 195.58 85.6774) (end 195.58 92.71) (width 0.25) (layer B.Cu) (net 6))
 (segment (start 201.93 99.06) (end 207.01 99.06) (width 0.25) (layer B.Cu) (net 6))
 (segment (start 195.58 92.71) (end 201.93 99.06) (width 0.25) (layer B.Cu) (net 6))
 (segment (start 190.427 90.8304) (end 195.58 85.6774) (width 0.25) (layer B.Cu) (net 6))
 (segment (start 175.2092 90.8304) (end 190.3762 90.8304) (width 0.25) (layer B.Cu) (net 6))
 (segment (start 163.83 79.4512) (end 175.2092 90.8304) (width 0.25) (layer B.Cu) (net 6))
 (segment (start 152.6032 79.4512) (end 163.8808 79.4512) (width 0.25) (layer B.Cu) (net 6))
 (segment (start 152.6032 79.4512) (end 150.5712 79.4512) (width 0.25) (layer F.Cu) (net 6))
 (segment (start 150.5712 79.4512) (end 146.05 74.93) (width 0.25) (layer F.Cu) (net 6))
 (segment (start 129.58 74.93) (end 127.2 72.55) (width 0.25) (layer F.Cu) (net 6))
 (segment (start 146.05 74.93) (end 129.58 74.93) (width 0.25) (layer F.Cu) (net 6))
 (segment (start 129.684999 89.959399) (end 129.684999 83.710999) (width 0.25) (layer F.Cu) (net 6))
 (segment (start 133.35 93.6244) (end 129.684999 89.959399) (width 0.25) (layer F.Cu) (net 6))
 (segment (start 127.2 81.226) (end 127.2 72.55) (width 0.25) (layer F.Cu) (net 6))
 (segment (start 129.684999 83.710999) (end 127.2 81.226) (width 0.25) (layer F.Cu) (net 6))
 (segment (start 127.4572 92.8116) (end 128.27 93.6244) (width 0.25) (layer B.Cu) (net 9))
 (segment (start 127.4572 91.367) (end 127.4572 92.8116) (width 0.25) (layer B.Cu) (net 9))
 (segment (start 126.5428 92.8116) (end 125.73 93.6244) (width 0.25) (layer B.Cu) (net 9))
 (segment (start 127.4572 92.8116) (end 126.5428 92.8116) (width 0.25) (layer B.Cu) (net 9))
 (segment (start 147.32 107.95) (end 150.368 107.95) (width 0.25) (layer F.Cu) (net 9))
 (segment (start 151.5872 106.7308) (end 151.5872 104.2924) (width 0.25) (layer F.Cu) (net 9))
 (segment (start 150.368 107.95) (end 151.5872 106.7308) (width 0.25) (layer F.Cu) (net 9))
 (segment (start 140.0556 107.95) (end 125.73 93.6244) (width 0.25) (layer B.Cu) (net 9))
 (segment (start 147.32 107.95) (end 140.0556 107.95) (width 0.25) (layer B.Cu) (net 9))
 (segment (start 144.7292 68.7832) (end 150.0632 68.7832) (width 0.25) (layer F.Cu) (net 28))
 (segment (start 152.6032 71.3232) (end 152.6032 74.3712) (width 0.25) (layer F.Cu) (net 28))
 (segment (start 150.0632 68.7832) (end 152.6032 71.3232) (width 0.25) (layer F.Cu) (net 28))
 (segment (start 154.9908 68.9356) (end 152.6032 71.3232) (width 0.25) (layer F.Cu) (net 28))
 (segment (start 165.608 68.9356) (end 154.9908 68.9356) (width 0.25) (layer F.Cu) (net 28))
 (segment (start 132.9944 91.44) (end 130.81 93.6244) (width 0.25) (layer B.Cu) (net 8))
 (segment (start 146.05 91.44) (end 132.9944 91.44) (width 0.25) (layer B.Cu) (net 8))
 (segment (start 146.05 93.98) (end 147.32 95.25) (width 0.25) (layer B.Cu) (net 8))
 (segment (start 146.05 91.44) (end 146.05 93.98) (width 0.25) (layer B.Cu) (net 8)))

